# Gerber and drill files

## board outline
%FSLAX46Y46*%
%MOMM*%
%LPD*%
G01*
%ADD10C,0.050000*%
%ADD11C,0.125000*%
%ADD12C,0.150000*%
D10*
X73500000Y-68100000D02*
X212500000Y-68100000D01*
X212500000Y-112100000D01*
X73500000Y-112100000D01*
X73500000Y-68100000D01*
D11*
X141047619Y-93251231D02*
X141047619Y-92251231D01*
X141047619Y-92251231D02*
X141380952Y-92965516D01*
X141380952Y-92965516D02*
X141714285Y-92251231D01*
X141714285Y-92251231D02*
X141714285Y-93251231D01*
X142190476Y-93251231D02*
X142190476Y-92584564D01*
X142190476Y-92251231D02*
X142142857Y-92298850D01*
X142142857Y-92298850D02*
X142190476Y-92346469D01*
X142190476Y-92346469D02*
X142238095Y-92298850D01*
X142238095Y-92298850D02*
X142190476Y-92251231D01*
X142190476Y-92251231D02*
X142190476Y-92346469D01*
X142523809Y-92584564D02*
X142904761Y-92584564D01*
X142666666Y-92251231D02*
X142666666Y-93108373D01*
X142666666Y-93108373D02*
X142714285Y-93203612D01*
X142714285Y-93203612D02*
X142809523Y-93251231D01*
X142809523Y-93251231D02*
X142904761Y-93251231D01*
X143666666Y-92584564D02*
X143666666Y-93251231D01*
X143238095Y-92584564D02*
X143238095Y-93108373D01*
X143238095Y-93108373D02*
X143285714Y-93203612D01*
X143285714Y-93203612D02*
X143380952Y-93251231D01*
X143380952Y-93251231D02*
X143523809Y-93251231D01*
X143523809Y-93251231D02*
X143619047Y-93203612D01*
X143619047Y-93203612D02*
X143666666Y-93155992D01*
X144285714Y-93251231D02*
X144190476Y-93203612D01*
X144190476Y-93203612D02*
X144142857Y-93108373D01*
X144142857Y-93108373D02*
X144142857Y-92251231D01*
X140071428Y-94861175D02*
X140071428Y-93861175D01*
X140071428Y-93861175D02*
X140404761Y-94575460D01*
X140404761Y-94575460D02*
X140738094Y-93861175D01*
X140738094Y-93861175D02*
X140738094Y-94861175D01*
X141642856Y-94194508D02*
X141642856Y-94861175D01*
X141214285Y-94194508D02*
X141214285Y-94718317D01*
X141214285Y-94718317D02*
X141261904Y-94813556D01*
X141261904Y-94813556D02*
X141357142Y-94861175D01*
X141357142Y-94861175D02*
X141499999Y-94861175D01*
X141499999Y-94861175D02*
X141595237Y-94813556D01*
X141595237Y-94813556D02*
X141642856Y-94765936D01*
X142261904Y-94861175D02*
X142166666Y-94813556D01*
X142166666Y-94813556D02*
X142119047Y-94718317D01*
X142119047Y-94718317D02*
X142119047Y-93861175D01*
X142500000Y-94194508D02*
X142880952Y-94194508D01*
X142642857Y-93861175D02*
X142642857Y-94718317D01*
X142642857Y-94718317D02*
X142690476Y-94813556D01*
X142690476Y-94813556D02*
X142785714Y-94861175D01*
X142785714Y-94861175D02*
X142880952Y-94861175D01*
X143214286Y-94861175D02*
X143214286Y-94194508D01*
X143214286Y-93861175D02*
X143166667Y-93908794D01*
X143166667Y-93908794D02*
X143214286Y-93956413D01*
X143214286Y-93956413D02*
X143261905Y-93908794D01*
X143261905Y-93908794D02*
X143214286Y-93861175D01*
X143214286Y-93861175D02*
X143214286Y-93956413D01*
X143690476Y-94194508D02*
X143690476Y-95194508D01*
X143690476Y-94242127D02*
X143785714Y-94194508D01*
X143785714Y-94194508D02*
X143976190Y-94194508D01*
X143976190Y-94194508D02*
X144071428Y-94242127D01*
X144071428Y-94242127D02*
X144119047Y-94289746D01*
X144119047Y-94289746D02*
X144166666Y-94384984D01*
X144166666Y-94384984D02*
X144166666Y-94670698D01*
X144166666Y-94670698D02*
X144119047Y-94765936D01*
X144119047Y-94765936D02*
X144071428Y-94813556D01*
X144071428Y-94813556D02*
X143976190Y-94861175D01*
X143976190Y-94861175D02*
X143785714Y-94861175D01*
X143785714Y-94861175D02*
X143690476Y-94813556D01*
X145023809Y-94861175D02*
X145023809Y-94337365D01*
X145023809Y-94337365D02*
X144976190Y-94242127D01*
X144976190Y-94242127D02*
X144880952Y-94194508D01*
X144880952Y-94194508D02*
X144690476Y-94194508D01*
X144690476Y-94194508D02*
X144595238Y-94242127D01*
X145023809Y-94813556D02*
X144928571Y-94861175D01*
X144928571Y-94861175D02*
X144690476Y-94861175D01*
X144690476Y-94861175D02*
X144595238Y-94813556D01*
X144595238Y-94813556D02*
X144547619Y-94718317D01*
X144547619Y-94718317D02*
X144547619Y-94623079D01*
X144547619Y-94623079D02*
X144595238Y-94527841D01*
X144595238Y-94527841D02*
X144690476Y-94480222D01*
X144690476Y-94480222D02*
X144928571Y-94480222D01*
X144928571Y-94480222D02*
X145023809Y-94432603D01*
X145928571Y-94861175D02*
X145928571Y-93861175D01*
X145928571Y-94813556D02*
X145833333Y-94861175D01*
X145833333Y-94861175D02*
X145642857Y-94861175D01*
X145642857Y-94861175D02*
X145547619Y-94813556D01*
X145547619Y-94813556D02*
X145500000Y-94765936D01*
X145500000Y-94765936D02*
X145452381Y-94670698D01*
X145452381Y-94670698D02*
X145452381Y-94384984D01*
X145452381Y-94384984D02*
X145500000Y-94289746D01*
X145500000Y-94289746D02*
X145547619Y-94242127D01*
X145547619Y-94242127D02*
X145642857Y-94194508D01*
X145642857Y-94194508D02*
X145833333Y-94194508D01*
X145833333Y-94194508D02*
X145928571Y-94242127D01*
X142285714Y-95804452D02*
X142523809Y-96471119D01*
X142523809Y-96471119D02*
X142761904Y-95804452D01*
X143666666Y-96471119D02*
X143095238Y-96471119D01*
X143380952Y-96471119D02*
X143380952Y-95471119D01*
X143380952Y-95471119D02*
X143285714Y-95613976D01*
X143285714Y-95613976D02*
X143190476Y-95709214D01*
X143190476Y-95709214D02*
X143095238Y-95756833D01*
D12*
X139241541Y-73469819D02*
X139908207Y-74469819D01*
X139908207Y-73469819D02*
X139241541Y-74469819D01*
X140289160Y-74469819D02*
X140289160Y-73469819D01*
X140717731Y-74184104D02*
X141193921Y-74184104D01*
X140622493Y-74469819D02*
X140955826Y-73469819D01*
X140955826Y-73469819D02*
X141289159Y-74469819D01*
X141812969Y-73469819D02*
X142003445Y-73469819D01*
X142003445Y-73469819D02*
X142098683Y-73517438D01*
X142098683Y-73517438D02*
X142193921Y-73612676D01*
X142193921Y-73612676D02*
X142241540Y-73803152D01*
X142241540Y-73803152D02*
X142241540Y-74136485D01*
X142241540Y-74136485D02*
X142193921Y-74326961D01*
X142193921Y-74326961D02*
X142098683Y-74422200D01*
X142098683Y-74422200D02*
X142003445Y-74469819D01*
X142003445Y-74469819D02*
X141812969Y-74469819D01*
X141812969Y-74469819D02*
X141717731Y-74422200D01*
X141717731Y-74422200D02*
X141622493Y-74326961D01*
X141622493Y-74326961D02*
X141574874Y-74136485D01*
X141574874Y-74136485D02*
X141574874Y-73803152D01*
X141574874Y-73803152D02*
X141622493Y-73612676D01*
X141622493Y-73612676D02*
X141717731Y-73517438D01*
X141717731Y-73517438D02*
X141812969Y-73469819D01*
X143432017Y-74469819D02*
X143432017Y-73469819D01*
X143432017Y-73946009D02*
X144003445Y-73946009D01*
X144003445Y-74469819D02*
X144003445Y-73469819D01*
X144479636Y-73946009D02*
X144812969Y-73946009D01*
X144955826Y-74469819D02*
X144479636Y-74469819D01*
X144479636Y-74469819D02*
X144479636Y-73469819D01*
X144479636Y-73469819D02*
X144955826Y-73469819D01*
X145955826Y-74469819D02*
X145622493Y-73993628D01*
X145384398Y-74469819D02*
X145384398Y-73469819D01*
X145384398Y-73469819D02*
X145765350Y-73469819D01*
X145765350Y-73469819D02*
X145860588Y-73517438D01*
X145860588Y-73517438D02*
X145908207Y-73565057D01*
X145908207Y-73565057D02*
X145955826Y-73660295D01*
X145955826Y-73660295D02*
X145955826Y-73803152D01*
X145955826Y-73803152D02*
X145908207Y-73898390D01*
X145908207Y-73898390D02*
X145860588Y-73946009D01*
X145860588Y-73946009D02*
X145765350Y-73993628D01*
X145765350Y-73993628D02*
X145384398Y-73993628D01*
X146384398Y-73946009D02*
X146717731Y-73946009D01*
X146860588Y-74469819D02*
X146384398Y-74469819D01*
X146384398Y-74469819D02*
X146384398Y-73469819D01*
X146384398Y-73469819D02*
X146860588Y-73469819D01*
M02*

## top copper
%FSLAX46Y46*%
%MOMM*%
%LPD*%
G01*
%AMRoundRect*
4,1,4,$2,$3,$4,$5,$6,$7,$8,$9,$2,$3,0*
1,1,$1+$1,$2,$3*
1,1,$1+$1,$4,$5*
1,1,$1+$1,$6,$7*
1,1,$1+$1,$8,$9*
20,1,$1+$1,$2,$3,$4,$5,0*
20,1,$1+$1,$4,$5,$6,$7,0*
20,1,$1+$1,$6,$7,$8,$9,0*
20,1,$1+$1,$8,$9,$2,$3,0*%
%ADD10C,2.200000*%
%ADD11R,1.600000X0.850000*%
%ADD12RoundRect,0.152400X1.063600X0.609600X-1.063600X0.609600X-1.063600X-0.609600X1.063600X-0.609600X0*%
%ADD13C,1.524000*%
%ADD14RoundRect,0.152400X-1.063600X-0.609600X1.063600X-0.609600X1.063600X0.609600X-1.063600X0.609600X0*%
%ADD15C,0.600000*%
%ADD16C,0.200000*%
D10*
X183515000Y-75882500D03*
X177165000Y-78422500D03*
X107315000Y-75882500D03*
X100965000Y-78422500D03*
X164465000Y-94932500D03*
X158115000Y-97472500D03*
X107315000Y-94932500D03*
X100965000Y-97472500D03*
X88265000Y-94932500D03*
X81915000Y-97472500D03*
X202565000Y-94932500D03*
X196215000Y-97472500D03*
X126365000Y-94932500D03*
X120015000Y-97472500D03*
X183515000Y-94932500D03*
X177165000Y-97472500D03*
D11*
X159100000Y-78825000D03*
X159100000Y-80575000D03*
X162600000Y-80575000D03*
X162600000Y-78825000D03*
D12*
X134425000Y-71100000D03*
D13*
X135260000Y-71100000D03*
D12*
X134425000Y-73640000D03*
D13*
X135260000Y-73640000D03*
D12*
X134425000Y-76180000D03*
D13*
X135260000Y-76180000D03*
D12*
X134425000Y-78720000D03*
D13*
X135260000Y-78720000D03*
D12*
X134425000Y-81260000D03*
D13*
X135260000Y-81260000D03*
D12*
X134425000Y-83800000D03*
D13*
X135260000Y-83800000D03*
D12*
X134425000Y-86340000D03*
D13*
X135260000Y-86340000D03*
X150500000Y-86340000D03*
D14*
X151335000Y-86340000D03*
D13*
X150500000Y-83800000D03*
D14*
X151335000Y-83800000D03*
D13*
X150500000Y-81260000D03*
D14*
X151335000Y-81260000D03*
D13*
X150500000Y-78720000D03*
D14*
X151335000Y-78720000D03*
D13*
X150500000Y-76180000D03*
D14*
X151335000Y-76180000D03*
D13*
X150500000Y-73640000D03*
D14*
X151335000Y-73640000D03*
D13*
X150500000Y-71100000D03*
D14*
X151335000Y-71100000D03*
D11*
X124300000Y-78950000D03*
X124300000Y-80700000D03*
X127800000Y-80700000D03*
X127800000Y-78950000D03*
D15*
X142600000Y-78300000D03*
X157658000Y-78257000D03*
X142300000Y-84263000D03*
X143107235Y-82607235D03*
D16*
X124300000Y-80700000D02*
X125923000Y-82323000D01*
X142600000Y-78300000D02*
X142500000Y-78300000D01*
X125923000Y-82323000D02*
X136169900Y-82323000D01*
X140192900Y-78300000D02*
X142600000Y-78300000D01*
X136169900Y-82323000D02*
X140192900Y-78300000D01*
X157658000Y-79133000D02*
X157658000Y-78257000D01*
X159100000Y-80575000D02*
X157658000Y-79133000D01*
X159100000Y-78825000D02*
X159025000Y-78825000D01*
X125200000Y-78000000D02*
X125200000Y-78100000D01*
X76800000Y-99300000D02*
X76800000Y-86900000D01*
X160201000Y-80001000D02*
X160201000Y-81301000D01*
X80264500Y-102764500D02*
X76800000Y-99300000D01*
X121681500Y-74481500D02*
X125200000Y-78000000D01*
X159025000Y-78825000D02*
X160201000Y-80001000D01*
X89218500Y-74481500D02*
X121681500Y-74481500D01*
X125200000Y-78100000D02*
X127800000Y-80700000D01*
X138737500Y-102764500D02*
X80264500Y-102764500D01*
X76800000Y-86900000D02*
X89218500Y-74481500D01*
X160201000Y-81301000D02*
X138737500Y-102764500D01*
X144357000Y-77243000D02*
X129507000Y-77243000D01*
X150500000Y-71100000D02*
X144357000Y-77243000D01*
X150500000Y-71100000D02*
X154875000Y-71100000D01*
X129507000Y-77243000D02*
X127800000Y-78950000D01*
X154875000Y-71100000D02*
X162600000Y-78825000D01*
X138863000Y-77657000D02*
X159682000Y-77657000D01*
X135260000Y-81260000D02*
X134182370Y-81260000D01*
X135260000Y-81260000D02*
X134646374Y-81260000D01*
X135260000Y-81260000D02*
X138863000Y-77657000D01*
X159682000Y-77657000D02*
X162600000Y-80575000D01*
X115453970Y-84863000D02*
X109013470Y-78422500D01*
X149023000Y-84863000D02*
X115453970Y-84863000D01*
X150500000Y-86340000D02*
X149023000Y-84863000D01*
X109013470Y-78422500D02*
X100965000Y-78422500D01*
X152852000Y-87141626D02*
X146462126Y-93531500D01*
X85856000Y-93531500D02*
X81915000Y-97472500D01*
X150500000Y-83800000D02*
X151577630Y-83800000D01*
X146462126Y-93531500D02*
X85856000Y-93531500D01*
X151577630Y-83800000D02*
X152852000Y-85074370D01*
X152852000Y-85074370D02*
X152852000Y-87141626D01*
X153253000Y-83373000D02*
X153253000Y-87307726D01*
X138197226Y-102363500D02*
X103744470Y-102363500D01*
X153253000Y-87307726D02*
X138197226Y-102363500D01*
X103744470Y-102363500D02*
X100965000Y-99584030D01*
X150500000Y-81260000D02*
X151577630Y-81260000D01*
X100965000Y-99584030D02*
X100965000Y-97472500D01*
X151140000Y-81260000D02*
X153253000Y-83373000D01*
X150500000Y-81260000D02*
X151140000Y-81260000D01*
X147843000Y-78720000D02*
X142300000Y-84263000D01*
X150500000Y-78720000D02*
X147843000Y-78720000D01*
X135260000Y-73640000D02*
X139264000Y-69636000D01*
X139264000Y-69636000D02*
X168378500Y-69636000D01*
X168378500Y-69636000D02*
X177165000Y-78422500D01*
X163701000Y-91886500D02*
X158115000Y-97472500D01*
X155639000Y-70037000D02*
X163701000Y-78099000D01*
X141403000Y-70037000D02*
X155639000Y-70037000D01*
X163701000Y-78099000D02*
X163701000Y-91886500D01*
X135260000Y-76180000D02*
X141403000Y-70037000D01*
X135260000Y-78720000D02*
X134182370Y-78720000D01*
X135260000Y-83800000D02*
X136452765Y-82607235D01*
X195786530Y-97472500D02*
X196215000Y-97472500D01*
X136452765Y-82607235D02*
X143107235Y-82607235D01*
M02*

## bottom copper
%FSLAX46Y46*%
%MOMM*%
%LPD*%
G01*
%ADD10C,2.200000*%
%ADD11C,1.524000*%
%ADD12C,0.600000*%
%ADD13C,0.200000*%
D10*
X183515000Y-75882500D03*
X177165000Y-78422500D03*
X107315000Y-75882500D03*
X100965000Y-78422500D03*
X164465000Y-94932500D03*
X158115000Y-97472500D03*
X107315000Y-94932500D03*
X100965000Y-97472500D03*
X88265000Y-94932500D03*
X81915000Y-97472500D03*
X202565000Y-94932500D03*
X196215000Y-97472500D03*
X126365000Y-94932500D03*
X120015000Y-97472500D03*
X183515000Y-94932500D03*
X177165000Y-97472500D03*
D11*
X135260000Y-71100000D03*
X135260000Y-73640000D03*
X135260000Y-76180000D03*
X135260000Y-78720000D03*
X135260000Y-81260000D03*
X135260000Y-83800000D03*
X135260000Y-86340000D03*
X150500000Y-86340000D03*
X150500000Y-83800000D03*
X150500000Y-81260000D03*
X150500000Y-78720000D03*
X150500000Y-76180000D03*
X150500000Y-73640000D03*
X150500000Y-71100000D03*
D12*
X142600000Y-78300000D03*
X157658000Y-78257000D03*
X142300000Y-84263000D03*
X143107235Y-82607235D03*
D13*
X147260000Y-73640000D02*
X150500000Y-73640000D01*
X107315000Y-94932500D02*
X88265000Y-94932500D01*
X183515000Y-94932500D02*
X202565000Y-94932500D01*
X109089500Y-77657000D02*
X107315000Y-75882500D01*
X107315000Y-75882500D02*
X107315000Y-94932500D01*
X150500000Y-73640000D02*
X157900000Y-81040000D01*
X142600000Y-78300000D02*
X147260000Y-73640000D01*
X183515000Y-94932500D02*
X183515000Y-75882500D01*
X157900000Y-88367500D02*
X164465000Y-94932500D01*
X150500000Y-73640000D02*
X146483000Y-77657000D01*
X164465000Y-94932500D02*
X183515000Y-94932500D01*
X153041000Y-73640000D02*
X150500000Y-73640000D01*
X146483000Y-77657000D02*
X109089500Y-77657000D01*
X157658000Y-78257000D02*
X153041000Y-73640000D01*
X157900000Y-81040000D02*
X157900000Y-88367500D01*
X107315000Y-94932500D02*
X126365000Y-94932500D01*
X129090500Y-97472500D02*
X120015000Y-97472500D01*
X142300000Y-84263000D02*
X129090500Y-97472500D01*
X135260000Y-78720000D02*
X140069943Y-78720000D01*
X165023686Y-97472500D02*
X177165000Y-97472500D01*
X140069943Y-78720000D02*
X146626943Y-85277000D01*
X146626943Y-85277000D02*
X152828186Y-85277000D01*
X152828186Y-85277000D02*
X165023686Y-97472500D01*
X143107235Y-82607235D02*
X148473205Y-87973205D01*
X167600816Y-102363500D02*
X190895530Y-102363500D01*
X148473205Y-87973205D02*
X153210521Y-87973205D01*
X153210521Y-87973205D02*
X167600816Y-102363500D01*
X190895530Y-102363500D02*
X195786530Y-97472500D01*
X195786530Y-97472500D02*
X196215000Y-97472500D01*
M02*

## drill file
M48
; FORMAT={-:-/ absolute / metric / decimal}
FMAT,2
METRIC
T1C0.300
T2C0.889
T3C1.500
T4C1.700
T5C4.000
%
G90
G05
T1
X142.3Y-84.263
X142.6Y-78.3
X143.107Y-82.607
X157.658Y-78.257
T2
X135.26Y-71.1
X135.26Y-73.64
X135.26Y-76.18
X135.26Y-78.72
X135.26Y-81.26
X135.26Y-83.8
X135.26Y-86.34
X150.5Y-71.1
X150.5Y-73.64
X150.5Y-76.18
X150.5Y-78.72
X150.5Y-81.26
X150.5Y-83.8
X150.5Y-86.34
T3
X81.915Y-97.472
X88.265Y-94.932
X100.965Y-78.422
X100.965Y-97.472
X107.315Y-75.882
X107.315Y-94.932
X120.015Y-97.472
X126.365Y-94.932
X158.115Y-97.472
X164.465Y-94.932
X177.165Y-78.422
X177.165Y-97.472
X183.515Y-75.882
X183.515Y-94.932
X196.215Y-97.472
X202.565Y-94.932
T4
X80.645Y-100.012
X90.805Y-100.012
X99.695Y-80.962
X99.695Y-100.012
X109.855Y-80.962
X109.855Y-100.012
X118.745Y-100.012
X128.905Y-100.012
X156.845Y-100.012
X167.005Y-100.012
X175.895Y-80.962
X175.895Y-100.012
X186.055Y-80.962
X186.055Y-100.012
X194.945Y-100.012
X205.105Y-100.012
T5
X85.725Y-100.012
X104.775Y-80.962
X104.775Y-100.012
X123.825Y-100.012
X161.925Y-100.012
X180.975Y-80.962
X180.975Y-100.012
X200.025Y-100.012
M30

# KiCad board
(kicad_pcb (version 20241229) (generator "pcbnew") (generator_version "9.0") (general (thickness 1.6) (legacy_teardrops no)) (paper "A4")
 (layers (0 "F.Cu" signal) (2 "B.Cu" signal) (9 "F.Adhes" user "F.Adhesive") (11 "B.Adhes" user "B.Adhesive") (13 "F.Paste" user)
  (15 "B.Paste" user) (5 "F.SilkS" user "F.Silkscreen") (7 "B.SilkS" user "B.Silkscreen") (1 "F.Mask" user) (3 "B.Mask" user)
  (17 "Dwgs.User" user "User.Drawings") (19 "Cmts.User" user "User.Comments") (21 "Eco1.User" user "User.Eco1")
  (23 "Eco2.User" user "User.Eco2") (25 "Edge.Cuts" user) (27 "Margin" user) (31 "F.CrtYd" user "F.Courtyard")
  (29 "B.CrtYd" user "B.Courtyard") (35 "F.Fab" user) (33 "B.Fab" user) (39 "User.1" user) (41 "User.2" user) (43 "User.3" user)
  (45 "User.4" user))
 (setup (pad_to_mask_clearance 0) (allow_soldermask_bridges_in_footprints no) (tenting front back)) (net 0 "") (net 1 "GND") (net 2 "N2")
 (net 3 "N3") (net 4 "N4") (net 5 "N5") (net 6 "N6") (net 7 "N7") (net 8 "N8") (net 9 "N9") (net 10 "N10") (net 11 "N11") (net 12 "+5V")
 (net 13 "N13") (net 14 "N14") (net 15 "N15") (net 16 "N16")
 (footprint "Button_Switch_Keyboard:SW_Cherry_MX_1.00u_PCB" (layer "F.Cu") (at 183.515 75.8825)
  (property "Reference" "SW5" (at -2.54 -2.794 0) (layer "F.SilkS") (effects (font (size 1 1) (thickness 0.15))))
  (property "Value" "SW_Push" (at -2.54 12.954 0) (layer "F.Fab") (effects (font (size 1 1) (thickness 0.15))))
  (pad "" np_thru_hole circle (at -7.62 5.08) (size 1.7 1.7) (drill 1.7) (layers "*.Cu" "*.Mask"))
  (pad "" np_thru_hole circle (at -2.54 5.08) (size 4 4) (drill 4) (layers "*.Cu" "*.Mask"))
  (pad "" np_thru_hole circle (at 2.54 5.08) (size 1.7 1.7) (drill 1.7) (layers "*.Cu" "*.Mask"))
  (pad "1" thru_hole circle (at 0 0) (size 2.2 2.2) (drill 1.5) (layers "*.Cu" "*.Mask") (remove_unused_layers no) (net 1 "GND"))
  (pad "2" thru_hole circle (at -6.35 2.54) (size 2.2 2.2) (drill 1.5) (layers "*.Cu" "*.Mask") (remove_unused_layers no) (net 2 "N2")))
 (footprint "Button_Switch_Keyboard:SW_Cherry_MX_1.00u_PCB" (layer "F.Cu") (at 107.315 75.8825)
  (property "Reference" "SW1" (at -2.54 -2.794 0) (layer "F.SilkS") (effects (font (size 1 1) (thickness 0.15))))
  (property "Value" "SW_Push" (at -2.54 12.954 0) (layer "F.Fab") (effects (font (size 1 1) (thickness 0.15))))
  (pad "" np_thru_hole circle (at -7.62 5.08) (size 1.7 1.7) (drill 1.7) (layers "*.Cu" "*.Mask"))
  (pad "" np_thru_hole circle (at -2.54 5.08) (size 4 4) (drill 4) (layers "*.Cu" "*.Mask"))
  (pad "" np_thru_hole circle (at 2.54 5.08) (size 1.7 1.7) (drill 1.7) (layers "*.Cu" "*.Mask"))
  (pad "1" thru_hole circle (at 0 0) (size 2.2 2.2) (drill 1.5) (layers "*.Cu" "*.Mask") (remove_unused_layers no) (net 1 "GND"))
  (pad "2" thru_hole circle (at -6.35 2.54) (size 2.2 2.2) (drill 1.5) (layers "*.Cu" "*.Mask") (remove_unused_layers no) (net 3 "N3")))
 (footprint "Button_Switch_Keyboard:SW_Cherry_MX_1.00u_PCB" (layer "F.Cu") (at 164.465 94.9325)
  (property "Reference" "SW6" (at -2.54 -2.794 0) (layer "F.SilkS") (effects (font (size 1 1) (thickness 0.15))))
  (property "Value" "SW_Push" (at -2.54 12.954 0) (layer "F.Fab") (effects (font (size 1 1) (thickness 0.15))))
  (pad "" np_thru_hole circle (at -7.62 5.08) (size 1.7 1.7) (drill 1.7) (layers "*.Cu" "*.Mask"))
  (pad "" np_thru_hole circle (at -2.54 5.08) (size 4 4) (drill 4) (layers "*.Cu" "*.Mask"))
  (pad "" np_thru_hole circle (at 2.54 5.08) (size 1.7 1.7) (drill 1.7) (layers "*.Cu" "*.Mask"))
  (pad "1" thru_hole circle (at 0 0) (size 2.2 2.2) (drill 1.5) (layers "*.Cu" "*.Mask") (remove_unused_layers no) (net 1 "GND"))
  (pad "2" thru_hole circle (at -6.35 2.54) (size 2.2 2.2) (drill 1.5) (layers "*.Cu" "*.Mask") (remove_unused_layers no) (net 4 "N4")))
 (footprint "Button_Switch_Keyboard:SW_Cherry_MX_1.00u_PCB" (layer "F.Cu") (at 107.315 94.9325)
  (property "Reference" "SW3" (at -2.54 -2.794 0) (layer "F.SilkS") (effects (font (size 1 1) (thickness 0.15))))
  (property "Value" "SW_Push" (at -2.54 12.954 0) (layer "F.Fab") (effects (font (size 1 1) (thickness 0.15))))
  (pad "" np_thru_hole circle (at -7.62 5.08) (size 1.7 1.7) (drill 1.7) (layers "*.Cu" "*.Mask"))
  (pad "" np_thru_hole circle (at -2.54 5.08) (size 4 4) (drill 4) (layers "*.Cu" "*.Mask"))
  (pad "" np_thru_hole circle (at 2.54 5.08) (size 1.7 1.7) (drill 1.7) (layers "*.Cu" "*.Mask"))
  (pad "1" thru_hole circle (at 0 0) (size 2.2 2.2) (drill 1.5) (layers "*.Cu" "*.Mask") (remove_unused_layers no) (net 1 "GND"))
  (pad "2" thru_hole circle (at -6.35 2.54) (size 2.2 2.2) (drill 1.5) (layers "*.Cu" "*.Mask") (remove_unused_layers no) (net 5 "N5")))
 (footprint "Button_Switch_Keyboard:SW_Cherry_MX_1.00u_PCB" (layer "F.Cu") (at 88.265 94.9325)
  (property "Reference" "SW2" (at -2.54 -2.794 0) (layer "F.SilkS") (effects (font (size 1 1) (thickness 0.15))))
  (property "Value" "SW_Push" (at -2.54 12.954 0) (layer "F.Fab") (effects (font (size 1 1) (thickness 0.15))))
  (pad "" np_thru_hole circle (at -7.62 5.08) (size 1.7 1.7) (drill 1.7) (layers "*.Cu" "*.Mask"))
  (pad "" np_thru_hole circle (at -2.54 5.08) (size 4 4) (drill 4) (layers "*.Cu" "*.Mask"))
  (pad "" np_thru_hole circle (at 2.54 5.08) (size 1.7 1.7) (drill 1.7) (layers "*.Cu" "*.Mask"))
  (pad "1" thru_hole circle (at 0 0) (size 2.2 2.2) (drill 1.5) (layers "*.Cu" "*.Mask") (remove_unused_layers no) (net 1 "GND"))
  (pad "2" thru_hole circle (at -6.35 2.54) (size 2.2 2.2) (drill 1.5) (layers "*.Cu" "*.Mask") (remove_unused_layers no) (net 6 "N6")))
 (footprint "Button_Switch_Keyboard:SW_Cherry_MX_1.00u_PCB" (layer "F.Cu") (at 202.565 94.9325)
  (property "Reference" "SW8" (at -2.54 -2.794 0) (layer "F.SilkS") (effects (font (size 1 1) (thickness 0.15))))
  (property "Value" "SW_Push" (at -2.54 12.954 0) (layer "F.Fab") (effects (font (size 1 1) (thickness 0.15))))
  (pad "" np_thru_hole circle (at -7.62 5.08) (size 1.7 1.7) (drill 1.7) (layers "*.Cu" "*.Mask"))
  (pad "" np_thru_hole circle (at -2.54 5.08) (size 4 4) (drill 4) (layers "*.Cu" "*.Mask"))
  (pad "" np_thru_hole circle (at 2.54 5.08) (size 1.7 1.7) (drill 1.7) (layers "*.Cu" "*.Mask"))
  (pad "1" thru_hole circle (at 0 0) (size 2.2 2.2) (drill 1.5) (layers "*.Cu" "*.Mask") (remove_unused_layers no) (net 1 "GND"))
  (pad "2" thru_hole circle (at -6.35 2.54) (size 2.2 2.2) (drill 1.5) (layers "*.Cu" "*.Mask") (remove_unused_layers no) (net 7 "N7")))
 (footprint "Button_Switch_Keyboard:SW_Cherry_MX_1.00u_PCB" (layer "F.Cu") (at 126.365 94.9325)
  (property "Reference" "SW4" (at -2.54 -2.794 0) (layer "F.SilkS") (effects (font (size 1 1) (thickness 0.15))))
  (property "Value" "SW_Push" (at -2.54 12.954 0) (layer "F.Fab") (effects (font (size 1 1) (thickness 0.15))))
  (pad "" np_thru_hole circle (at -7.62 5.08) (size 1.7 1.7) (drill 1.7) (layers "*.Cu" "*.Mask"))
  (pad "" np_thru_hole circle (at -2.54 5.08) (size 4 4) (drill 4) (layers "*.Cu" "*.Mask"))
  (pad "" np_thru_hole circle (at 2.54 5.08) (size 1.7 1.7) (drill 1.7) (layers "*.Cu" "*.Mask"))
  (pad "1" thru_hole circle (at 0 0) (size 2.2 2.2) (drill 1.5) (layers "*.Cu" "*.Mask") (remove_unused_layers no) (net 1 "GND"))
  (pad "2" thru_hole circle (at -6.35 2.54) (size 2.2 2.2) (drill 1.5) (layers "*.Cu" "*.Mask") (remove_unused_layers no) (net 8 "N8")))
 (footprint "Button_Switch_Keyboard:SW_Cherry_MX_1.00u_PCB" (layer "F.Cu") (at 183.515 94.9325)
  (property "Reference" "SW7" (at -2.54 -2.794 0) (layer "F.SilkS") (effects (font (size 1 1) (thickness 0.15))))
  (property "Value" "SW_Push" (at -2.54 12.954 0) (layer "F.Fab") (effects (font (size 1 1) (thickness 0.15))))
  (pad "" np_thru_hole circle (at -7.62 5.08) (size 1.7 1.7) (drill 1.7) (layers "*.Cu" "*.Mask"))
  (pad "" np_thru_hole circle (at -2.54 5.08) (size 4 4) (drill 4) (layers "*.Cu" "*.Mask"))
  (pad "" np_thru_hole circle (at 2.54 5.08) (size 1.7 1.7) (drill 1.7) (layers "*.Cu" "*.Mask"))
  (pad "1" thru_hole circle (at 0 0) (size 2.2 2.2) (drill 1.5) (layers "*.Cu" "*.Mask") (remove_unused_layers no) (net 1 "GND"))
  (pad "2" thru_hole circle (at -6.35 2.54) (size 2.2 2.2) (drill 1.5) (layers "*.Cu" "*.Mask") (remove_unused_layers no) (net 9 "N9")))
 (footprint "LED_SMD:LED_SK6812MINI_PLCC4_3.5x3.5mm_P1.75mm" (layer "F.Cu") (at 160.85 79.7)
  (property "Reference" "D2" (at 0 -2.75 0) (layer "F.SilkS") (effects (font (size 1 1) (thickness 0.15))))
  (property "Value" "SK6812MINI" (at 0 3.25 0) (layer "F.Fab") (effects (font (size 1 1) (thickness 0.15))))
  (pad "1" smd rect (at -1.75 -0.875) (size 1.6 0.85) (layers "F.Cu" "F.Mask" "F.Paste") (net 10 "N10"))
  (pad "2" smd rect (at -1.75 0.875) (size 1.6 0.85) (layers "F.Cu" "F.Mask" "F.Paste") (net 1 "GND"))
  (pad "3" smd rect (at 1.75 0.875) (size 1.6 0.85) (layers "F.Cu" "F.Mask" "F.Paste") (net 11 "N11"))
  (pad "4" smd rect (at 1.75 -0.875) (size 1.6 0.85) (layers "F.Cu" "F.Mask" "F.Paste") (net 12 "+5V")))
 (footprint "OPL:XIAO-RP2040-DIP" (layer "F.Cu") (at 142.88 78.72)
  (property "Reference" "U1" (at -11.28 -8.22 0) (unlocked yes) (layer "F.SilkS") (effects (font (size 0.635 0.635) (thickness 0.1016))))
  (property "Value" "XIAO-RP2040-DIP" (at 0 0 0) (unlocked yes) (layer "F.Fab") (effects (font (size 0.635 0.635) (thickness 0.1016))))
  (pad "1" smd roundrect (at -8.455 -7.62 180) (size 2.432 1.524) (layers "F.Cu" "F.Mask") (roundrect_rratio 0.1) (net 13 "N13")
   (thermal_bridge_angle 45))
  (pad "1" thru_hole circle (at -7.62 -7.62 180) (size 1.524 1.524) (drill 0.889) (layers "*.Cu" "*.Mask") (remove_unused_layers no)
   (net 13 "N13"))
  (pad "2" smd roundrect (at -8.455 -5.08 180) (size 2.432 1.524) (layers "F.Cu" "F.Mask") (roundrect_rratio 0.1) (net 2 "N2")
   (thermal_bridge_angle 45))
  (pad "2" thru_hole circle (at -7.62 -5.08 180) (size 1.524 1.524) (drill 0.889) (layers "*.Cu" "*.Mask") (remove_unused_layers no)
   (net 2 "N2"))
  (pad "3" smd roundrect (at -8.455 -2.54 180) (size 2.432 1.524) (layers "F.Cu" "F.Mask") (roundrect_rratio 0.1) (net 4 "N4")
   (thermal_bridge_angle 45))
  (pad "3" thru_hole circle (at -7.62 -2.54 180) (size 1.524 1.524) (drill 0.889) (layers "*.Cu" "*.Mask") (remove_unused_layers no)
   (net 4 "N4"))
  (pad "4" smd roundrect (at -8.455 0 180) (size 2.432 1.524) (layers "F.Cu" "F.Mask") (roundrect_rratio 0.1) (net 9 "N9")
   (thermal_bridge_angle 45))
  (pad "4" thru_hole circle (at -7.62 0 180) (size 1.524 1.524) (drill 0.889) (layers "*.Cu" "*.Mask") (remove_unused_layers no)
   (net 9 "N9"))
  (pad "5" smd roundrect (at -8.455 2.54 180) (size 2.432 1.524) (layers "F.Cu" "F.Mask") (roundrect_rratio 0.1) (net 11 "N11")
   (thermal_bridge_angle 45))
  (pad "5" thru_hole circle (at -7.62 2.54 180) (size 1.524 1.524) (drill 0.889) (layers "*.Cu" "*.Mask") (remove_unused_layers no)
   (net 11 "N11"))
  (pad "6" smd roundrect (at -8.455 5.08 180) (size 2.432 1.524) (layers "F.Cu" "F.Mask") (roundrect_rratio 0.1) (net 7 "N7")
   (thermal_bridge_angle 45))
  (pad "6" thru_hole circle (at -7.62 5.08 180) (size 1.524 1.524) (drill 0.889) (layers "*.Cu" "*.Mask") (remove_unused_layers no)
   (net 7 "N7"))
  (pad "7" smd roundrect (at -8.455 7.62 180) (size 2.432 1.524) (layers "F.Cu" "F.Mask") (roundrect_rratio 0.1) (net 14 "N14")
   (thermal_bridge_angle 45))
  (pad "7" thru_hole circle (at -7.62 7.62 180) (size 1.524 1.524) (drill 0.889) (layers "*.Cu" "*.Mask") (remove_unused_layers no)
   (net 14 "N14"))
  (pad "8" thru_hole circle (at 7.62 7.62) (size 1.524 1.524) (drill 0.889) (layers "*.Cu" "*.Mask") (remove_unused_layers no) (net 3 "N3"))
  (pad "8" smd roundrect (at 8.455 7.62) (size 2.432 1.524) (layers "F.Cu" "F.Mask") (roundrect_rratio 0.1) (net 3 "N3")
   (thermal_bridge_angle 45))
  (pad "9" thru_hole circle (at 7.62 5.08) (size 1.524 1.524) (drill 0.889) (layers "*.Cu" "*.Mask") (remove_unused_layers no) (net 6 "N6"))
  (pad "9" smd roundrect (at 8.455 5.08) (size 2.432 1.524) (layers "F.Cu" "F.Mask") (roundrect_rratio 0.1) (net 6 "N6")
   (thermal_bridge_angle 45))
  (pad "10" thru_hole circle (at 7.62 2.54) (size 1.524 1.524) (drill 0.889) (layers "*.Cu" "*.Mask") (remove_unused_layers no) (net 5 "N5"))
  (pad "10" smd roundrect (at 8.455 2.54) (size 2.432 1.524) (layers "F.Cu" "F.Mask") (roundrect_rratio 0.1) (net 5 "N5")
   (thermal_bridge_angle 45))
  (pad "11" thru_hole circle (at 7.62 0) (size 1.524 1.524) (drill 0.889) (layers "*.Cu" "*.Mask") (remove_unused_layers no) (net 8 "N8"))
  (pad "11" smd roundrect (at 8.455 0) (size 2.432 1.524) (layers "F.Cu" "F.Mask") (roundrect_rratio 0.1) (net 8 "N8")
   (thermal_bridge_angle 45))
  (pad "12" thru_hole circle (at 7.62 -2.54) (size 1.524 1.524) (drill 0.889) (layers "*.Cu" "*.Mask") (remove_unused_layers no)
   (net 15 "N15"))
  (pad "12" smd roundrect (at 8.455 -2.54) (size 2.432 1.524) (layers "F.Cu" "F.Mask") (roundrect_rratio 0.1) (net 15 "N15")
   (thermal_bridge_angle 45))
  (pad "13" thru_hole circle (at 7.62 -5.08) (size 1.524 1.524) (drill 0.889) (layers "*.Cu" "*.Mask") (remove_unused_layers no)
   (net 1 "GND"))
  (pad "13" smd roundrect (at 8.455 -5.08) (size 2.432 1.524) (layers "F.Cu" "F.Mask") (roundrect_rratio 0.1) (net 1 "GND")
   (thermal_bridge_angle 45))
  (pad "14" thru_hole circle (at 7.62 -7.62) (size 1.524 1.524) (drill 0.889) (layers "*.Cu" "*.Mask") (remove_unused_layers no)
   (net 12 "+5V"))
  (pad "14" smd roundrect (at 8.455 -7.62) (size 2.432 1.524) (layers "F.Cu" "F.Mask") (roundrect_rratio 0.1) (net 12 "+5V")
   (thermal_bridge_angle 45)))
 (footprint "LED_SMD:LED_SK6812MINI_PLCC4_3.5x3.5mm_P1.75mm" (layer "F.Cu") (at 126.05 79.825)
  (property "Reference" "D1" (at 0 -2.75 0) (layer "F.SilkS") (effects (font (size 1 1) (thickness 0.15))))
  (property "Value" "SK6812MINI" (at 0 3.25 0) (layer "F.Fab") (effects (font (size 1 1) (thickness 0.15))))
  (pad "1" smd rect (at -1.75 -0.875) (size 1.6 0.85) (layers "F.Cu" "F.Mask" "F.Paste") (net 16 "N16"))
  (pad "2" smd rect (at -1.75 0.875) (size 1.6 0.85) (layers "F.Cu" "F.Mask" "F.Paste") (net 1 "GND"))
  (pad "3" smd rect (at 1.75 0.875) (size 1.6 0.85) (layers "F.Cu" "F.Mask" "F.Paste") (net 10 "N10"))
  (pad "4" smd rect (at 1.75 -0.875) (size 1.6 0.85) (layers "F.Cu" "F.Mask" "F.Paste") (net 12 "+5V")))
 (gr_rect (start 73.5 68.1) (end 212.5 112.1) (stroke (width 0.05) (type default)) (fill no) (layer "Edge.Cuts"))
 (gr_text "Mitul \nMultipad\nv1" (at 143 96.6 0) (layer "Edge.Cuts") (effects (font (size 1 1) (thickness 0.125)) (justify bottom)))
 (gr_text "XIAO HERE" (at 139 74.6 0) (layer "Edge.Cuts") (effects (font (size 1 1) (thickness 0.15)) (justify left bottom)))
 (segment (start 124.3 80.7) (end 125.923 82.323) (width 0.2) (layer "F.Cu") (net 1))
 (segment (start 142.6 78.3) (end 142.5 78.3) (width 0.2) (layer "F.Cu") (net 1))
 (segment (start 125.923 82.323) (end 136.1699 82.323) (width 0.2) (layer "F.Cu") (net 1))
 (segment (start 140.1929 78.3) (end 142.6 78.3) (width 0.2) (layer "F.Cu") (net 1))
 (segment (start 136.1699 82.323) (end 140.1929 78.3) (width 0.2) (layer "F.Cu") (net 1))
 (segment (start 157.658 79.133) (end 157.658 78.257) (width 0.2) (layer "F.Cu") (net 1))
 (segment (start 159.1 80.575) (end 157.658 79.133) (width 0.2) (layer "F.Cu") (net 1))
 (via (at 142.6 78.3) (size 0.6) (drill 0.3) (layers "F.Cu" "B.Cu") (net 1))
 (via (at 157.658 78.257) (size 0.6) (drill 0.3) (layers "F.Cu" "B.Cu") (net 1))
 (segment (start 147.26 73.64) (end 150.5 73.64) (width 0.2) (layer "B.Cu") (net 1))
 (segment (start 107.315 94.9325) (end 88.265 94.9325) (width 0.2) (layer "B.Cu") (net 1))
 (segment (start 183.515 94.9325) (end 202.565 94.9325) (width 0.2) (layer "B.Cu") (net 1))
 (segment (start 109.0895 77.657) (end 107.315 75.8825) (width 0.2) (layer "B.Cu") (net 1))
 (segment (start 107.315 75.8825) (end 107.315 94.9325) (width 0.2) (layer "B.Cu") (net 1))
 (segment (start 150.5 73.64) (end 157.9 81.04) (width 0.2) (layer "B.Cu") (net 1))
 (segment (start 142.6 78.3) (end 147.26 73.64) (width 0.2) (layer "B.Cu") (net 1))
 (segment (start 183.515 94.9325) (end 183.515 75.8825) (width 0.2) (layer "B.Cu") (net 1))
 (segment (start 157.9 88.3675) (end 164.465 94.9325) (width 0.2) (layer "B.Cu") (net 1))
 (segment (start 150.5 73.64) (end 146.483 77.657) (width 0.2) (layer "B.Cu") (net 1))
 (segment (start 164.465 94.9325) (end 183.515 94.9325) (width 0.2) (layer "B.Cu") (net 1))
 (segment (start 153.041 73.64) (end 150.5 73.64) (width 0.2) (layer "B.Cu") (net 1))
 (segment (start 146.483 77.657) (end 109.0895 77.657) (width 0.2) (layer "B.Cu") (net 1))
 (segment (start 157.658 78.257) (end 153.041 73.64) (width 0.2) (layer "B.Cu") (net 1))
 (segment (start 157.9 81.04) (end 157.9 88.3675) (width 0.2) (layer "B.Cu") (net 1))
 (segment (start 107.315 94.9325) (end 126.365 94.9325) (width 0.2) (layer "B.Cu") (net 1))
 (segment (start 159.1 78.825) (end 159.025 78.825) (width 0.2) (layer "F.Cu") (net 10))
 (segment (start 125.2 78) (end 125.2 78.1) (width 0.2) (layer "F.Cu") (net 10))
 (segment (start 76.8 99.3) (end 76.8 86.9) (width 0.2) (layer "F.Cu") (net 10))
 (segment (start 160.201 80.001) (end 160.201 81.301) (width 0.2) (layer "F.Cu") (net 10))
 (segment (start 80.2645 102.7645) (end 76.8 99.3) (width 0.2) (layer "F.Cu") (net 10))
 (segment (start 121.6815 74.4815) (end 125.2 78) (width 0.2) (layer "F.Cu") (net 10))
 (segment (start 159.025 78.825) (end 160.201 80.001) (width 0.2) (layer "F.Cu") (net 10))
 (segment (start 89.2185 74.4815) (end 121.6815 74.4815) (width 0.2) (layer "F.Cu") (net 10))
 (segment (start 125.2 78.1) (end 127.8 80.7) (width 0.2) (layer "F.Cu") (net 10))
 (segment (start 138.7375 102.7645) (end 80.2645 102.7645) (width 0.2) (layer "F.Cu") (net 10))
 (segment (start 76.8 86.9) (end 89.2185 74.4815) (width 0.2) (layer "F.Cu") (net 10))
 (segment (start 160.201 81.301) (end 138.7375 102.7645) (width 0.2) (layer "F.Cu") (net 10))
 (segment (start 144.357 77.243) (end 129.507 77.243) (width 0.2) (layer "F.Cu") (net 12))
 (segment (start 150.5 71.1) (end 144.357 77.243) (width 0.2) (layer "F.Cu") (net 12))
 (segment (start 150.5 71.1) (end 154.875 71.1) (width 0.2) (layer "F.Cu") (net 12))
 (segment (start 129.507 77.243) (end 127.8 78.95) (width 0.2) (layer "F.Cu") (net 12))
 (segment (start 154.875 71.1) (end 162.6 78.825) (width 0.2) (layer "F.Cu") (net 12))
 (segment (start 138.863 77.657) (end 159.682 77.657) (width 0.2) (layer "F.Cu") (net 11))
 (segment (start 135.26 81.26) (end 134.18237 81.26) (width 0.2) (layer "F.Cu") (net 11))
 (segment (start 135.26 81.26) (end 134.646374 81.26) (width 0.2) (layer "F.Cu") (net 11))
 (segment (start 135.26 81.26) (end 138.863 77.657) (width 0.2) (layer "F.Cu") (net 11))
 (segment (start 159.682 77.657) (end 162.6 80.575) (width 0.2) (layer "F.Cu") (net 11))
 (segment (start 115.45397 84.863) (end 109.01347 78.4225) (width 0.2) (layer "F.Cu") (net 3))
 (segment (start 149.023 84.863) (end 115.45397 84.863) (width 0.2) (layer "F.Cu") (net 3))
 (segment (start 150.5 86.34) (end 149.023 84.863) (width 0.2) (layer "F.Cu") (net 3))
 (segment (start 109.01347 78.4225) (end 100.965 78.4225) (width 0.2) (layer "F.Cu") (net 3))
 (segment (start 152.852 87.141626) (end 146.462126 93.5315) (width 0.2) (layer "F.Cu") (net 6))
 (segment (start 85.856 93.5315) (end 81.915 97.4725) (width 0.2) (layer "F.Cu") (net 6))
 (segment (start 150.5 83.8) (end 151.57763 83.8) (width 0.2) (layer "F.Cu") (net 6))
 (segment (start 146.462126 93.5315) (end 85.856 93.5315) (width 0.2) (layer "F.Cu") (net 6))
 (segment (start 151.57763 83.8) (end 152.852 85.07437) (width 0.2) (layer "F.Cu") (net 6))
 (segment (start 152.852 85.07437) (end 152.852 87.141626) (width 0.2) (layer "F.Cu") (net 6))
 (segment (start 153.253 83.373) (end 153.253 87.307726) (width 0.2) (layer "F.Cu") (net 5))
 (segment (start 138.197226 102.3635) (end 103.74447 102.3635) (width 0.2) (layer "F.Cu") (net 5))
 (segment (start 153.253 87.307726) (end 138.197226 102.3635) (width 0.2) (layer "F.Cu") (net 5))
 (segment (start 103.74447 102.3635) (end 100.965 99.58403) (width 0.2) (layer "F.Cu") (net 5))
 (segment (start 150.5 81.26) (end 151.57763 81.26) (width 0.2) (layer "F.Cu") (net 5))
 (segment (start 100.965 99.58403) (end 100.965 97.4725) (width 0.2) (layer "F.Cu") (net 5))
 (segment (start 151.14 81.26) (end 153.253 83.373) (width 0.2) (layer "F.Cu") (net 5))
 (segment (start 150.5 81.26) (end 151.14 81.26) (width 0.2) (layer "F.Cu") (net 5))
 (segment (start 147.843 78.72) (end 142.3 84.263) (width 0.2) (layer "F.Cu") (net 8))
 (segment (start 150.5 78.72) (end 147.843 78.72) (width 0.2) (layer "F.Cu") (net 8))
 (via (at 142.3 84.263) (size 0.6) (drill 0.3) (layers "F.Cu" "B.Cu") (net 8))
 (segment (start 129.0905 97.4725) (end 120.015 97.4725) (width 0.2) (layer "B.Cu") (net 8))
 (segment (start 142.3 84.263) (end 129.0905 97.4725) (width 0.2) (layer "B.Cu") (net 8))
 (segment (start 135.26 73.64) (end 139.264 69.636) (width 0.2) (layer "F.Cu") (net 2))
 (segment (start 139.264 69.636) (end 168.3785 69.636) (width 0.2) (layer "F.Cu") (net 2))
 (segment (start 168.3785 69.636) (end 177.165 78.4225) (width 0.2) (layer "F.Cu") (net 2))
 (segment (start 163.701 91.8865) (end 158.115 97.4725) (width 0.2) (layer "F.Cu") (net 4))
 (segment (start 155.639 70.037) (end 163.701 78.099) (width 0.2) (layer "F.Cu") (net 4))
 (segment (start 141.403 70.037) (end 155.639 70.037) (width 0.2) (layer "F.Cu") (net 4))
 (segment (start 163.701 78.099) (end 163.701 91.8865) (width 0.2) (layer "F.Cu") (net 4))
 (segment (start 135.26 76.18) (end 141.403 70.037) (width 0.2) (layer "F.Cu") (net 4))
 (segment (start 135.26 78.72) (end 134.18237 78.72) (width 0.2) (layer "F.Cu") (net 9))
 (segment (start 135.26 78.72) (end 140.069943 78.72) (width 0.2) (layer "B.Cu") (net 9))
 (segment (start 165.023686 97.4725) (end 177.165 97.4725) (width 0.2) (layer "B.Cu") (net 9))
 (segment (start 140.069943 78.72) (end 146.626943 85.277) (width 0.2) (layer "B.Cu") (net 9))
 (segment (start 146.626943 85.277) (end 152.828186 85.277) (width 0.2) (layer "B.Cu") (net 9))
 (segment (start 152.828186 85.277) (end 165.023686 97.4725) (width 0.2) (layer "B.Cu") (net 9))
 (segment (start 135.26 83.8) (end 136.452765 82.607235) (width 0.2) (layer "F.Cu") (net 7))
 (segment (start 195.78653 97.4725) (end 196.215 97.4725) (width 0.2) (layer "F.Cu") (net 7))
 (segment (start 136.452765 82.607235) (end 143.107235 82.607235) (width 0.2) (layer "F.Cu") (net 7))
 (via (at 143.107235 82.607235) (size 0.6) (drill 0.3) (layers "F.Cu" "B.Cu") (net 7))
 (segment (start 143.107235 82.607235) (end 148.473205 87.973205) (width 0.2) (layer "B.Cu") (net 7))
 (segment (start 167.600816 102.3635) (end 190.89553 102.3635) (width 0.2) (layer "B.Cu") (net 7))
 (segment (start 148.473205 87.973205) (end 153.210521 87.973205) (width 0.2) (layer "B.Cu") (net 7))
 (segment (start 153.210521 87.973205) (end 167.600816 102.3635) (width 0.2) (layer "B.Cu") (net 7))
 (segment (start 190.89553 102.3635) (end 195.78653 97.4725) (width 0.2) (layer "B.Cu") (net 7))
 (segment (start 195.78653 97.4725) (end 196.215 97.4725) (width 0.2) (layer "B.Cu") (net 7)))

